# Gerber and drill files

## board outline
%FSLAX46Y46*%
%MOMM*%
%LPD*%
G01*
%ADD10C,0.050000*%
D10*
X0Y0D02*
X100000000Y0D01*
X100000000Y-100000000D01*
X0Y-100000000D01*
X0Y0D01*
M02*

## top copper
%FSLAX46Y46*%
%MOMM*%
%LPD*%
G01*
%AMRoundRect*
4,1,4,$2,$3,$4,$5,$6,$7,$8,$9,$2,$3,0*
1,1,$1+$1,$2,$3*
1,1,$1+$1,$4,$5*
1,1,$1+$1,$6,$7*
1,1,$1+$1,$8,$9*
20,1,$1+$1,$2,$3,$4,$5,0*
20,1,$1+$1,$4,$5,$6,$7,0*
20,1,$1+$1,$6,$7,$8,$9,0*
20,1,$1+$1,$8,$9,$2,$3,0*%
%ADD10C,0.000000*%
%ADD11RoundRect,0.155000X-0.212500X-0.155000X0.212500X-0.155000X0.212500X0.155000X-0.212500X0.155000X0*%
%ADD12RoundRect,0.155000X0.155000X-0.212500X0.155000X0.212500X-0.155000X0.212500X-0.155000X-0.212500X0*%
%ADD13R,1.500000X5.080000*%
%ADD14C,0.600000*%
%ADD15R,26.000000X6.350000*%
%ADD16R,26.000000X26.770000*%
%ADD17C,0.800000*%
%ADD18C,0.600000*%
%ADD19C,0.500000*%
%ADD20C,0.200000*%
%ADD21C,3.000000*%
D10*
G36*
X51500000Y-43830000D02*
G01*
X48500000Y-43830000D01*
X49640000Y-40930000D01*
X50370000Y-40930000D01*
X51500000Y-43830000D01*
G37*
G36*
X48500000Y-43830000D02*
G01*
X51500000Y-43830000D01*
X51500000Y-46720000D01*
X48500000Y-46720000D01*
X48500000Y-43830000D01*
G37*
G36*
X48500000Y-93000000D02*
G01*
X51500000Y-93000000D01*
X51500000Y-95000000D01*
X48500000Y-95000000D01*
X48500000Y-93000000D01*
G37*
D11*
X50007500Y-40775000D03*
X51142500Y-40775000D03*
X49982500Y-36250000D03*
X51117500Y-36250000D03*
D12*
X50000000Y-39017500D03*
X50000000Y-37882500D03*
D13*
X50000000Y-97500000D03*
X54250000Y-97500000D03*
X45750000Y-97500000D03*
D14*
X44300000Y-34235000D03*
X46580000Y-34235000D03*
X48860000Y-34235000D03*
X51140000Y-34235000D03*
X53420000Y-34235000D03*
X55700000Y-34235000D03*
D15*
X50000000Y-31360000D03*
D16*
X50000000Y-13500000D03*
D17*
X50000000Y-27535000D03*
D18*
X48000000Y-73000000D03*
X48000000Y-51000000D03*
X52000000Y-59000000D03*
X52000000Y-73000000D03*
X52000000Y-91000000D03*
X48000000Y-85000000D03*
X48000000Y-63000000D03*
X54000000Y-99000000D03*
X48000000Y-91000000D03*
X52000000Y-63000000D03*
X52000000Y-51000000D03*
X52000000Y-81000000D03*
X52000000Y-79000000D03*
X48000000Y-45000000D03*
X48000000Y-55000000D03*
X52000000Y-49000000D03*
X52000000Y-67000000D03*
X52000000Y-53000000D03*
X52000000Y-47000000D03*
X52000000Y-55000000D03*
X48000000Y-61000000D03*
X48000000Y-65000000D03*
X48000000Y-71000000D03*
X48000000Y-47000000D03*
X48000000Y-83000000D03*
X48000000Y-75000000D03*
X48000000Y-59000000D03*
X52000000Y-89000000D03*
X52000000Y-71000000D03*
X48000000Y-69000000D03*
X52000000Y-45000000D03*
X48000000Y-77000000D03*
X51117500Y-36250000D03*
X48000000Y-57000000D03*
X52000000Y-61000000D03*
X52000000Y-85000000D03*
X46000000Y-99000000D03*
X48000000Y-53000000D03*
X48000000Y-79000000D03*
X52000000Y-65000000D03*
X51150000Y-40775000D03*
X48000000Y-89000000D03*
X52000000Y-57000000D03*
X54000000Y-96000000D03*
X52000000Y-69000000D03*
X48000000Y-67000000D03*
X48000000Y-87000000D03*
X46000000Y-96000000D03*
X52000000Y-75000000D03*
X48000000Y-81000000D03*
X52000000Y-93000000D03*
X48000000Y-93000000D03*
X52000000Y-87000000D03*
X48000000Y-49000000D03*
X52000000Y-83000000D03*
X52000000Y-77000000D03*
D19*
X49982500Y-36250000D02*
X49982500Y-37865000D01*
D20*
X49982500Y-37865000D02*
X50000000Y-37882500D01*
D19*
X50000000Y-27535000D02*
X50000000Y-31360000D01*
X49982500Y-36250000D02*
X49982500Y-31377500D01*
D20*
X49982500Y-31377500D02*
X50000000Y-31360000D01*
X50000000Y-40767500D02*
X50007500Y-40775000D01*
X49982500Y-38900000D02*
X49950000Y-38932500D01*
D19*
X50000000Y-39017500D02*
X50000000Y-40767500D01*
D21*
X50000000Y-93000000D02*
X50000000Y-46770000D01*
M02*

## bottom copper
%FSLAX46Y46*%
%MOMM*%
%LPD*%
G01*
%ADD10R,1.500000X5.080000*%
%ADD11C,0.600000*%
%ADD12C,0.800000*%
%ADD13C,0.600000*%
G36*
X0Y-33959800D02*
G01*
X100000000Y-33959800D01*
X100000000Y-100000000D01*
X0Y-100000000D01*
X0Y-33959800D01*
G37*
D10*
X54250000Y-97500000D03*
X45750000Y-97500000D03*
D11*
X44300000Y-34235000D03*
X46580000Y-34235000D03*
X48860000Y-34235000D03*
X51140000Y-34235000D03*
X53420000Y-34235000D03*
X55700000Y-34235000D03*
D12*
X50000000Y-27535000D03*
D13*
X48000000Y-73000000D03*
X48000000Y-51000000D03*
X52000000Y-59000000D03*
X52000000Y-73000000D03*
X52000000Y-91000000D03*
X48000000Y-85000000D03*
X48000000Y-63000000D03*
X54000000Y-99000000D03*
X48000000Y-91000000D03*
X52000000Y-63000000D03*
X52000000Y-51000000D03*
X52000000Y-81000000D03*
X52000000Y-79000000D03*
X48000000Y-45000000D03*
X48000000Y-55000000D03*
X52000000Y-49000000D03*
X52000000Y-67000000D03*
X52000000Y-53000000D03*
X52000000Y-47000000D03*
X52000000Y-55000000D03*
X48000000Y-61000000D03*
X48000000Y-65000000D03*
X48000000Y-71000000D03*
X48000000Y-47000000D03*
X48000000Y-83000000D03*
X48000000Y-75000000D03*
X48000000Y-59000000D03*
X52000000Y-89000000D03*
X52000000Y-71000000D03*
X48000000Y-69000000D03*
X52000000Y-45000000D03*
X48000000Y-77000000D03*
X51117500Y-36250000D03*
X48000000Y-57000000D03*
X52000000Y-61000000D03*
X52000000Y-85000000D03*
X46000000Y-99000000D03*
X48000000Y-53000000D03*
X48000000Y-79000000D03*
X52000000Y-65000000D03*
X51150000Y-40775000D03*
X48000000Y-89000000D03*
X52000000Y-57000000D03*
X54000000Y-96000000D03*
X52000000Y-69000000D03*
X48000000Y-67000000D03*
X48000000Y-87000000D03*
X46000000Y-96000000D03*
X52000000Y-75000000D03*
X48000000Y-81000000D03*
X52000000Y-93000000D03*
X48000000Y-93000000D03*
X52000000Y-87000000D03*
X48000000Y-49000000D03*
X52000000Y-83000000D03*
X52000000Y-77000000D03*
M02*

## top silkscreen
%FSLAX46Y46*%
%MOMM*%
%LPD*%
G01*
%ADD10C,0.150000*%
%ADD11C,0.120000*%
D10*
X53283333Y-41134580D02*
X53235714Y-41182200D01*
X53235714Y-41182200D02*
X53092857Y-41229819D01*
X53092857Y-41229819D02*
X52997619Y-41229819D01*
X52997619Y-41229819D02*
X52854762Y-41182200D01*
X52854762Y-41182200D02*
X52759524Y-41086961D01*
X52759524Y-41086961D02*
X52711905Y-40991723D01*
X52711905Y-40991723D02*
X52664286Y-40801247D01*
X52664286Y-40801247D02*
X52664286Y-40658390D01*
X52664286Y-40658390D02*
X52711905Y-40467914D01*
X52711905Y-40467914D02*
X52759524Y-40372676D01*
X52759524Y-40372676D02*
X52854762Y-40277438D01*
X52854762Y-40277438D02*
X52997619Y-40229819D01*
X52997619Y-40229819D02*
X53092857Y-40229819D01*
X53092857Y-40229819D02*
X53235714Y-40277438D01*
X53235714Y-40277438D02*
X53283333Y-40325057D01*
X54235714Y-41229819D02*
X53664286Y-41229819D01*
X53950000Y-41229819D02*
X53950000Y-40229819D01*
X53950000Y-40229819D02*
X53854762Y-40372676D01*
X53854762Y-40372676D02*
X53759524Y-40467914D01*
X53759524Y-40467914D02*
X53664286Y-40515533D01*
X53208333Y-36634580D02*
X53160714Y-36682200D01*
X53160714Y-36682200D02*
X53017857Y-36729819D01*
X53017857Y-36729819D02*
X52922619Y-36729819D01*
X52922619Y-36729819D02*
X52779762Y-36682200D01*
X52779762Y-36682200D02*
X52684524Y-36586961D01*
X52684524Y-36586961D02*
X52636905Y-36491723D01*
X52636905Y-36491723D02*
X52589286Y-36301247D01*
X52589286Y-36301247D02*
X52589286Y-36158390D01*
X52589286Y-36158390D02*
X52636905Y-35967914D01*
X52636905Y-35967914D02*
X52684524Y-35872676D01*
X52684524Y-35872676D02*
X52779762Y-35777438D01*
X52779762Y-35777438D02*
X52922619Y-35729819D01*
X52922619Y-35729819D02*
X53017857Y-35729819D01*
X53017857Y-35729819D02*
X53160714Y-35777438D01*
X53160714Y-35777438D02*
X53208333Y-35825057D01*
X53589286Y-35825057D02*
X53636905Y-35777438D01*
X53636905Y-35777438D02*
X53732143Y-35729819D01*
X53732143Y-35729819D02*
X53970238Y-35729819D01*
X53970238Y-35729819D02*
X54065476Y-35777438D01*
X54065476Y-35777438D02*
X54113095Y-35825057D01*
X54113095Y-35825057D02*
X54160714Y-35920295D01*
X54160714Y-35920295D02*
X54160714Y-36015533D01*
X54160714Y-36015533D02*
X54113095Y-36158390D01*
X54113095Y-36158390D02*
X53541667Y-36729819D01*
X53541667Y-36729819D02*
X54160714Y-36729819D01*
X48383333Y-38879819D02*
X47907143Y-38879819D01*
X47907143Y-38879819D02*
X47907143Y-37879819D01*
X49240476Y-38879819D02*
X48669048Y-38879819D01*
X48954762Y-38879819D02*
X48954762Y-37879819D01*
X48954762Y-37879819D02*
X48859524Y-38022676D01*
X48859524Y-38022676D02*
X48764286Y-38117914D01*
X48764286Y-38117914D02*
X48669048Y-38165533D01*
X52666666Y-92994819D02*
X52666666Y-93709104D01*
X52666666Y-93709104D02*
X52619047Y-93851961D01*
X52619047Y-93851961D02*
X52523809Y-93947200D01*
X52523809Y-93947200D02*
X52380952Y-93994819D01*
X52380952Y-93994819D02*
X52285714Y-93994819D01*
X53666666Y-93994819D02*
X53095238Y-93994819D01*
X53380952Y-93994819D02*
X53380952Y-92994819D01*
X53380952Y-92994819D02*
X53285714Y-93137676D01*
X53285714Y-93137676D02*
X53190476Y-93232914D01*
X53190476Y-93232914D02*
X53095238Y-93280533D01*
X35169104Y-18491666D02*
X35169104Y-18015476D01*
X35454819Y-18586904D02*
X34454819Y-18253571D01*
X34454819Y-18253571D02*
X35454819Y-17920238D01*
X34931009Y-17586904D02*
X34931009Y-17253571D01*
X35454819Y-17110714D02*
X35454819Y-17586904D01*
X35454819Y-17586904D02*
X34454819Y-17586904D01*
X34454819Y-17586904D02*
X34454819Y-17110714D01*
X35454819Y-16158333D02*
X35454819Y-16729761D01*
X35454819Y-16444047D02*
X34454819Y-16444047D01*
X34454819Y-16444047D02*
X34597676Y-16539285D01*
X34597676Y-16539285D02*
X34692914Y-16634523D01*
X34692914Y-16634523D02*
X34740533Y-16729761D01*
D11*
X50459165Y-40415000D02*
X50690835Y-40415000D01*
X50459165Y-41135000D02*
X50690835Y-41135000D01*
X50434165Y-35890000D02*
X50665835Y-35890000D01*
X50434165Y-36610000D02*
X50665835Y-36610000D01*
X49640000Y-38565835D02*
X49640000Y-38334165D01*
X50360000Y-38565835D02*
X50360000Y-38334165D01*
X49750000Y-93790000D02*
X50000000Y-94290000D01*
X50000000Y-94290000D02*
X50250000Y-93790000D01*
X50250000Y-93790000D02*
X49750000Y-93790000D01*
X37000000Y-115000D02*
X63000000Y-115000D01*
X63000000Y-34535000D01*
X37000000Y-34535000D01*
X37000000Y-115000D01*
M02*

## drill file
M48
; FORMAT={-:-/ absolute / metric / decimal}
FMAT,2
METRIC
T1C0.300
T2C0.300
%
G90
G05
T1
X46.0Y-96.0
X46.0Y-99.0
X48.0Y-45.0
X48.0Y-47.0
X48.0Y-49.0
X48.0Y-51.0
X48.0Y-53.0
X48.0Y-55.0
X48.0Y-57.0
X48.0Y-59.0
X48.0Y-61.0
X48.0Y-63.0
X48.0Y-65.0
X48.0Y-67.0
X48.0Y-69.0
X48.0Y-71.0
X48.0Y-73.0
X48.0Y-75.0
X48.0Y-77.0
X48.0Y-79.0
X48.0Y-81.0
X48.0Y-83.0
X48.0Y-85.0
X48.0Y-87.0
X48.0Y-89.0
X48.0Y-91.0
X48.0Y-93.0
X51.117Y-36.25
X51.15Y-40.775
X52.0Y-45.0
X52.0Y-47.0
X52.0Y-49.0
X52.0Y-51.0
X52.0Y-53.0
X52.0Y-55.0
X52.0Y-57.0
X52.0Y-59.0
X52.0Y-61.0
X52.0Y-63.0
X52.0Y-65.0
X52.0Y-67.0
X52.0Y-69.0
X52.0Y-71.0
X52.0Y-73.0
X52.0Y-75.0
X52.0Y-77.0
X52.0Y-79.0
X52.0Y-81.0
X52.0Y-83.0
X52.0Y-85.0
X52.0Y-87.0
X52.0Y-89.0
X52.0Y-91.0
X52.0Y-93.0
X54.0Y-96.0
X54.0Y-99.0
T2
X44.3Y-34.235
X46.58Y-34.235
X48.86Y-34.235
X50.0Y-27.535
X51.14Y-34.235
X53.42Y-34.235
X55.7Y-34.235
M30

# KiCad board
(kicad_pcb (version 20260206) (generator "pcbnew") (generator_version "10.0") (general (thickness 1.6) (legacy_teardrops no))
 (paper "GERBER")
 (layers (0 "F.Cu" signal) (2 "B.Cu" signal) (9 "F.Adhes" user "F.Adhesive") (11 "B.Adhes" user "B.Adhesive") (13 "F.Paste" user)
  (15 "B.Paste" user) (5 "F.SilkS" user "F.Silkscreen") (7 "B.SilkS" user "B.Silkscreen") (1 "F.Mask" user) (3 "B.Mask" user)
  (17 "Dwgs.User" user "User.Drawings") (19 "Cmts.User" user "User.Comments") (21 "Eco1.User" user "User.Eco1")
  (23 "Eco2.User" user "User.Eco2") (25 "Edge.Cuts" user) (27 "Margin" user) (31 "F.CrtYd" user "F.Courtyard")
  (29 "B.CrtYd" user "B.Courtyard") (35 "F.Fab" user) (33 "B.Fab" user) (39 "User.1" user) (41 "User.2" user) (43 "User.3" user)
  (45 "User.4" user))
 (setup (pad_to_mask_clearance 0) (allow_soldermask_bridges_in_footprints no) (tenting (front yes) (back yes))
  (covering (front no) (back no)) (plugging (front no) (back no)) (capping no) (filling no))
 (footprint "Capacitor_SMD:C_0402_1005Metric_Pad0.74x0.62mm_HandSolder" (layer "F.Cu") (at 50.575 40.775)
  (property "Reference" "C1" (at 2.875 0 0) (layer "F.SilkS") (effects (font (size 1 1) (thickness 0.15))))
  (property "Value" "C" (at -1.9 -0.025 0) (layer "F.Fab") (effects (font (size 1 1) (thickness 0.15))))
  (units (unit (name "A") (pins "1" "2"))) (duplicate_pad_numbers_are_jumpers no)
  (fp_line (start -0.115835 -0.36) (end 0.115835 -0.36) (stroke (width 0.12) (type solid)) (layer "F.SilkS"))
  (fp_line (start -0.115835 0.36) (end 0.115835 0.36) (stroke (width 0.12) (type solid)) (layer "F.SilkS"))
  (pad "1" smd roundrect (at -0.5675 0) (size 0.735 0.62) (layers "F.Cu" "F.Mask" "F.Paste") (roundrect_rratio 0.25) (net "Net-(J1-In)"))
  (pad "2" smd roundrect (at 0.5675 0) (size 0.735 0.62) (layers "F.Cu" "F.Mask" "F.Paste") (roundrect_rratio 0.25) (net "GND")))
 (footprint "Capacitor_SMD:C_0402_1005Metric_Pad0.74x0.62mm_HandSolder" (layer "F.Cu") (at 50.55 36.25)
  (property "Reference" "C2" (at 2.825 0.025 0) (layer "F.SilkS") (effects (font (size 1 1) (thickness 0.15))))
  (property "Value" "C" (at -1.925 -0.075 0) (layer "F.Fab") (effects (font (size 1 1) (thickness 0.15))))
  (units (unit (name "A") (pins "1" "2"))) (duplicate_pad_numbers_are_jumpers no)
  (fp_line (start -0.115835 -0.36) (end 0.115835 -0.36) (stroke (width 0.12) (type solid)) (layer "F.SilkS"))
  (fp_line (start -0.115835 0.36) (end 0.115835 0.36) (stroke (width 0.12) (type solid)) (layer "F.SilkS"))
  (pad "1" smd roundrect (at -0.5675 0) (size 0.735 0.62) (layers "F.Cu" "F.Mask" "F.Paste") (roundrect_rratio 0.25) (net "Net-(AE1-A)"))
  (pad "2" smd roundrect (at 0.5675 0) (size 0.735 0.62) (layers "F.Cu" "F.Mask" "F.Paste") (roundrect_rratio 0.25) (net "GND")))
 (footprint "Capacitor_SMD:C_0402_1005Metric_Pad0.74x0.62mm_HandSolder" (layer "F.Cu") (at 50 38.45 90)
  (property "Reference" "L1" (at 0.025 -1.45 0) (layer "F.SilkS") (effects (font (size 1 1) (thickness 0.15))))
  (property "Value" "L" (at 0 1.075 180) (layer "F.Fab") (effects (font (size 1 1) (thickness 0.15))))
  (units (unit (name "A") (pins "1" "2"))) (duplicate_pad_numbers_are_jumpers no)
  (fp_line (start -0.115835 -0.36) (end 0.115835 -0.36) (stroke (width 0.12) (type solid)) (layer "F.SilkS"))
  (fp_line (start -0.115835 0.36) (end 0.115835 0.36) (stroke (width 0.12) (type solid)) (layer "F.SilkS"))
  (pad "1" smd roundrect (at -0.5675 0 90) (size 0.735 0.62) (layers "F.Cu" "F.Mask" "F.Paste") (roundrect_rratio 0.25) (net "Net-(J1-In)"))
  (pad "2" smd roundrect (at 0.5675 0 90) (size 0.735 0.62) (layers "F.Cu" "F.Mask" "F.Paste") (roundrect_rratio 0.25) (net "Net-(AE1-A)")))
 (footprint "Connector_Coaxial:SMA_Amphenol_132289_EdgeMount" (layer "F.Cu") (at 50 97.5 -90)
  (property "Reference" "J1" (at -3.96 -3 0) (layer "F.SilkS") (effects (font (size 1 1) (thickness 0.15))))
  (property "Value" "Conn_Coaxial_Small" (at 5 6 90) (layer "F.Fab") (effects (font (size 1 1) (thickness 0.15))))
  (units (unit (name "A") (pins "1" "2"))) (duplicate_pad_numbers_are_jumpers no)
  (fp_line (start -3.71 0.25) (end -3.21 0) (stroke (width 0.12) (type solid)) (layer "F.SilkS"))
  (fp_line (start -3.21 0) (end -3.71 -0.25) (stroke (width 0.12) (type solid)) (layer "F.SilkS"))
  (fp_line (start -3.71 -0.25) (end -3.71 0.25) (stroke (width 0.12) (type solid)) (layer "F.SilkS"))
  (pad "1" smd rect (at 0 0) (size 1.5 5.08) (layers "F.Cu" "F.Mask" "F.Paste") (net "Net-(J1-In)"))
  (pad "2" smd rect (at 0 -4.25) (size 1.5 5.08) (layers "F.Cu" "F.Mask" "F.Paste") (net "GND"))
  (pad "2" smd rect (at 0 -4.25) (size 1.5 5.08) (layers "B.Cu" "B.Mask" "B.Paste") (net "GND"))
  (pad "2" smd rect (at 0 4.25) (size 1.5 5.08) (layers "F.Cu" "F.Mask" "F.Paste") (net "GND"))
  (pad "2" smd rect (at 0 4.25) (size 1.5 5.08) (layers "B.Cu" "B.Mask" "B.Paste") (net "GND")))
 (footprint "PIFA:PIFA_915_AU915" (layer "F.Cu") (at 37 34.535 90)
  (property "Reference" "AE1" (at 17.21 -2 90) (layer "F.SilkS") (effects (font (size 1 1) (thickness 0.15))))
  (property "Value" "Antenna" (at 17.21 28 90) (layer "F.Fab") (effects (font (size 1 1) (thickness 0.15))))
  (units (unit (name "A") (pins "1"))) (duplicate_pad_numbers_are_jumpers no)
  (fp_rect (start 0 0) (end 34.42 26) (stroke (width 0.12) (type solid)) (fill no) (layer "F.SilkS"))
  (pad "1" thru_hole circle (at 0.3 7.3 90) (size 0.6 0.6) (drill 0.3) (layers "*.Cu" "*.Mask") (remove_unused_layers no) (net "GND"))
  (pad "1" thru_hole circle (at 0.3 9.58 90) (size 0.6 0.6) (drill 0.3) (layers "*.Cu" "*.Mask") (remove_unused_layers no) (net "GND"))
  (pad "1" thru_hole circle (at 0.3 11.86 90) (size 0.6 0.6) (drill 0.3) (layers "*.Cu" "*.Mask") (remove_unused_layers no) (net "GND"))
  (pad "1" thru_hole circle (at 0.3 14.14 90) (size 0.6 0.6) (drill 0.3) (layers "*.Cu" "*.Mask") (remove_unused_layers no) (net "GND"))
  (pad "1" thru_hole circle (at 0.3 16.42 90) (size 0.6 0.6) (drill 0.3) (layers "*.Cu" "*.Mask") (remove_unused_layers no) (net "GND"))
  (pad "1" thru_hole circle (at 0.3 18.7 90) (size 0.6 0.6) (drill 0.3) (layers "*.Cu" "*.Mask") (remove_unused_layers no) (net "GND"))
  (pad "1" smd rect (at 3.175 13 90) (size 6.35 26) (layers "F.Cu" "F.Mask") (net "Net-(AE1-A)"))
  (pad "1" smd rect (at 21.035 13 90) (size 26.77 26) (layers "F.Cu" "F.Mask") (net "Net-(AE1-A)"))
  (pad "2" thru_hole circle (at 7 13 90) (size 0.8 0.8) (drill 0.3) (layers "*.Cu" "*.Mask") (remove_unused_layers no) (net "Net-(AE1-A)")))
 (gr_poly
  (pts (xy 48.5 43.83) (xy 49.64 40.93) (xy 50.37 40.93) (xy 51.5 43.83)) (stroke (width 0) (type solid)) (fill yes) (layer "F.Cu")
  (net "Net-(J1-In)"))
 (gr_rect (start 48.5 43.83) (end 51.5 46.72) (stroke (width 0) (type solid)) (fill yes) (layer "F.Cu") (net "Net-(J1-In)"))
 (gr_rect (start 48.5 93) (end 51.5 95) (stroke (width 0) (type solid)) (fill yes) (layer "F.Cu") (net "Net-(J1-In)"))
 (gr_rect (start 0 33.9598) (end 100 100) (stroke (width 0) (type solid)) (fill yes) (layer "B.Cu") (net "GND"))
 (gr_rect (start 0 0) (end 100 100) (stroke (width 0.05) (type solid)) (fill no) (layer "Edge.Cuts"))
 (segment (start 49.9825 36.25) (end 49.9825 37.865) (width 0.5) (layer "F.Cu") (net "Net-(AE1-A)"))
 (segment (start 49.9825 37.865) (end 50 37.8825) (width 0.2) (layer "F.Cu") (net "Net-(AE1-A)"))
 (segment (start 50 27.535) (end 50 31.36) (width 0.5) (layer "F.Cu") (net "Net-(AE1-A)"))
 (segment (start 49.9825 36.25) (end 49.9825 31.3775) (width 0.5) (layer "F.Cu") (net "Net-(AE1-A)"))
 (segment (start 49.9825 31.3775) (end 50 31.36) (width 0.2) (layer "F.Cu") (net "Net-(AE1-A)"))
 (via (at 48 73) (size 0.6) (drill 0.3) (layers "F.Cu" "B.Cu") (free yes) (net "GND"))
 (via (at 48 51) (size 0.6) (drill 0.3) (layers "F.Cu" "B.Cu") (free yes) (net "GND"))
 (via (at 52 59) (size 0.6) (drill 0.3) (layers "F.Cu" "B.Cu") (free yes) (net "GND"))
 (via (at 52 73) (size 0.6) (drill 0.3) (layers "F.Cu" "B.Cu") (free yes) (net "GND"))
 (via (at 52 91) (size 0.6) (drill 0.3) (layers "F.Cu" "B.Cu") (free yes) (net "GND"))
 (via (at 48 85) (size 0.6) (drill 0.3) (layers "F.Cu" "B.Cu") (free yes) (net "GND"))
 (via (at 48 63) (size 0.6) (drill 0.3) (layers "F.Cu" "B.Cu") (free yes) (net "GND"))
 (via (at 54 99) (size 0.6) (drill 0.3) (layers "F.Cu" "B.Cu") (free yes) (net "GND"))
 (via (at 48 91) (size 0.6) (drill 0.3) (layers "F.Cu" "B.Cu") (free yes) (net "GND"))
 (via (at 52 63) (size 0.6) (drill 0.3) (layers "F.Cu" "B.Cu") (free yes) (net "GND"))
 (via (at 52 51) (size 0.6) (drill 0.3) (layers "F.Cu" "B.Cu") (free yes) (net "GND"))
 (via (at 52 81) (size 0.6) (drill 0.3) (layers "F.Cu" "B.Cu") (free yes) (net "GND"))
 (via (at 52 79) (size 0.6) (drill 0.3) (layers "F.Cu" "B.Cu") (free yes) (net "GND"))
 (via (at 48 45) (size 0.6) (drill 0.3) (layers "F.Cu" "B.Cu") (free yes) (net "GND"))
 (via (at 48 55) (size 0.6) (drill 0.3) (layers "F.Cu" "B.Cu") (free yes) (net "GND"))
 (via (at 52 49) (size 0.6) (drill 0.3) (layers "F.Cu" "B.Cu") (free yes) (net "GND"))
 (via (at 52 67) (size 0.6) (drill 0.3) (layers "F.Cu" "B.Cu") (free yes) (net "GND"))
 (via (at 52 53) (size 0.6) (drill 0.3) (layers "F.Cu" "B.Cu") (free yes) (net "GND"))
 (via (at 52 47) (size 0.6) (drill 0.3) (layers "F.Cu" "B.Cu") (free yes) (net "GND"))
 (via (at 52 55) (size 0.6) (drill 0.3) (layers "F.Cu" "B.Cu") (free yes) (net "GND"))
 (via (at 48 61) (size 0.6) (drill 0.3) (layers "F.Cu" "B.Cu") (free yes) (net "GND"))
 (via (at 48 65) (size 0.6) (drill 0.3) (layers "F.Cu" "B.Cu") (free yes) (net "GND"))
 (via (at 48 71) (size 0.6) (drill 0.3) (layers "F.Cu" "B.Cu") (free yes) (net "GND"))
 (via (at 48 47) (size 0.6) (drill 0.3) (layers "F.Cu" "B.Cu") (free yes) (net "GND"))
 (via (at 48 83) (size 0.6) (drill 0.3) (layers "F.Cu" "B.Cu") (free yes) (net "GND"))
 (via (at 48 75) (size 0.6) (drill 0.3) (layers "F.Cu" "B.Cu") (free yes) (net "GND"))
 (via (at 48 59) (size 0.6) (drill 0.3) (layers "F.Cu" "B.Cu") (free yes) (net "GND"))
 (via (at 52 89) (size 0.6) (drill 0.3) (layers "F.Cu" "B.Cu") (free yes) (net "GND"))
 (via (at 52 71) (size 0.6) (drill 0.3) (layers "F.Cu" "B.Cu") (free yes) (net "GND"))
 (via (at 48 69) (size 0.6) (drill 0.3) (layers "F.Cu" "B.Cu") (free yes) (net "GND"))
 (via (at 52 45) (size 0.6) (drill 0.3) (layers "F.Cu" "B.Cu") (free yes) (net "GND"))
 (via (at 48 77) (size 0.6) (drill 0.3) (layers "F.Cu" "B.Cu") (free yes) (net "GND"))
 (via (at 51.1175 36.25) (size 0.6) (drill 0.3) (layers "F.Cu" "B.Cu") (free yes) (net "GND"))
 (via (at 48 57) (size 0.6) (drill 0.3) (layers "F.Cu" "B.Cu") (free yes) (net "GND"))
 (via (at 52 61) (size 0.6) (drill 0.3) (layers "F.Cu" "B.Cu") (free yes) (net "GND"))
 (via (at 52 85) (size 0.6) (drill 0.3) (layers "F.Cu" "B.Cu") (free yes) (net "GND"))
 (via (at 46 99) (size 0.6) (drill 0.3) (layers "F.Cu" "B.Cu") (free yes) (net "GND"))
 (via (at 48 53) (size 0.6) (drill 0.3) (layers "F.Cu" "B.Cu") (free yes) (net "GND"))
 (via (at 48 79) (size 0.6) (drill 0.3) (layers "F.Cu" "B.Cu") (free yes) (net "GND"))
 (via (at 52 65) (size 0.6) (drill 0.3) (layers "F.Cu" "B.Cu") (free yes) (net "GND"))
 (via (at 51.15 40.775) (size 0.6) (drill 0.3) (layers "F.Cu" "B.Cu") (free yes) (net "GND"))
 (via (at 48 89) (size 0.6) (drill 0.3) (layers "F.Cu" "B.Cu") (free yes) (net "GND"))
 (via (at 52 57) (size 0.6) (drill 0.3) (layers "F.Cu" "B.Cu") (free yes) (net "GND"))
 (via (at 54 96) (size 0.6) (drill 0.3) (layers "F.Cu" "B.Cu") (free yes) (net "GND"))
 (via (at 52 69) (size 0.6) (drill 0.3) (layers "F.Cu" "B.Cu") (free yes) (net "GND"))
 (via (at 48 67) (size 0.6) (drill 0.3) (layers "F.Cu" "B.Cu") (free yes) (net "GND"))
 (via (at 48 87) (size 0.6) (drill 0.3) (layers "F.Cu" "B.Cu") (free yes) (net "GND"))
 (via (at 46 96) (size 0.6) (drill 0.3) (layers "F.Cu" "B.Cu") (free yes) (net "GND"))
 (via (at 52 75) (size 0.6) (drill 0.3) (layers "F.Cu" "B.Cu") (free yes) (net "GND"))
 (via (at 48 81) (size 0.6) (drill 0.3) (layers "F.Cu" "B.Cu") (free yes) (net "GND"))
 (via (at 52 93) (size 0.6) (drill 0.3) (layers "F.Cu" "B.Cu") (free yes) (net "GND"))
 (via (at 48 93) (size 0.6) (drill 0.3) (layers "F.Cu" "B.Cu") (free yes) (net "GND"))
 (via (at 52 87) (size 0.6) (drill 0.3) (layers "F.Cu" "B.Cu") (free yes) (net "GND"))
 (via (at 48 49) (size 0.6) (drill 0.3) (layers "F.Cu" "B.Cu") (free yes) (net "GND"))
 (via (at 52 83) (size 0.6) (drill 0.3) (layers "F.Cu" "B.Cu") (free yes) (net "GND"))
 (via (at 52 77) (size 0.6) (drill 0.3) (layers "F.Cu" "B.Cu") (free yes) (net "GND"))
 (segment (start 50 40.7675) (end 50.0075 40.775) (width 0.2) (layer "F.Cu") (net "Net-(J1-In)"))
 (segment (start 49.9825 38.9) (end 49.95 38.9325) (width 0.2) (layer "F.Cu") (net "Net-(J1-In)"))
 (segment (start 50 39.0175) (end 50 40.7675) (width 0.5) (layer "F.Cu") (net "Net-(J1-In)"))
 (segment (start 50 93) (end 50 46.77) (width 3) (layer "F.Cu") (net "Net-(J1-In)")))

